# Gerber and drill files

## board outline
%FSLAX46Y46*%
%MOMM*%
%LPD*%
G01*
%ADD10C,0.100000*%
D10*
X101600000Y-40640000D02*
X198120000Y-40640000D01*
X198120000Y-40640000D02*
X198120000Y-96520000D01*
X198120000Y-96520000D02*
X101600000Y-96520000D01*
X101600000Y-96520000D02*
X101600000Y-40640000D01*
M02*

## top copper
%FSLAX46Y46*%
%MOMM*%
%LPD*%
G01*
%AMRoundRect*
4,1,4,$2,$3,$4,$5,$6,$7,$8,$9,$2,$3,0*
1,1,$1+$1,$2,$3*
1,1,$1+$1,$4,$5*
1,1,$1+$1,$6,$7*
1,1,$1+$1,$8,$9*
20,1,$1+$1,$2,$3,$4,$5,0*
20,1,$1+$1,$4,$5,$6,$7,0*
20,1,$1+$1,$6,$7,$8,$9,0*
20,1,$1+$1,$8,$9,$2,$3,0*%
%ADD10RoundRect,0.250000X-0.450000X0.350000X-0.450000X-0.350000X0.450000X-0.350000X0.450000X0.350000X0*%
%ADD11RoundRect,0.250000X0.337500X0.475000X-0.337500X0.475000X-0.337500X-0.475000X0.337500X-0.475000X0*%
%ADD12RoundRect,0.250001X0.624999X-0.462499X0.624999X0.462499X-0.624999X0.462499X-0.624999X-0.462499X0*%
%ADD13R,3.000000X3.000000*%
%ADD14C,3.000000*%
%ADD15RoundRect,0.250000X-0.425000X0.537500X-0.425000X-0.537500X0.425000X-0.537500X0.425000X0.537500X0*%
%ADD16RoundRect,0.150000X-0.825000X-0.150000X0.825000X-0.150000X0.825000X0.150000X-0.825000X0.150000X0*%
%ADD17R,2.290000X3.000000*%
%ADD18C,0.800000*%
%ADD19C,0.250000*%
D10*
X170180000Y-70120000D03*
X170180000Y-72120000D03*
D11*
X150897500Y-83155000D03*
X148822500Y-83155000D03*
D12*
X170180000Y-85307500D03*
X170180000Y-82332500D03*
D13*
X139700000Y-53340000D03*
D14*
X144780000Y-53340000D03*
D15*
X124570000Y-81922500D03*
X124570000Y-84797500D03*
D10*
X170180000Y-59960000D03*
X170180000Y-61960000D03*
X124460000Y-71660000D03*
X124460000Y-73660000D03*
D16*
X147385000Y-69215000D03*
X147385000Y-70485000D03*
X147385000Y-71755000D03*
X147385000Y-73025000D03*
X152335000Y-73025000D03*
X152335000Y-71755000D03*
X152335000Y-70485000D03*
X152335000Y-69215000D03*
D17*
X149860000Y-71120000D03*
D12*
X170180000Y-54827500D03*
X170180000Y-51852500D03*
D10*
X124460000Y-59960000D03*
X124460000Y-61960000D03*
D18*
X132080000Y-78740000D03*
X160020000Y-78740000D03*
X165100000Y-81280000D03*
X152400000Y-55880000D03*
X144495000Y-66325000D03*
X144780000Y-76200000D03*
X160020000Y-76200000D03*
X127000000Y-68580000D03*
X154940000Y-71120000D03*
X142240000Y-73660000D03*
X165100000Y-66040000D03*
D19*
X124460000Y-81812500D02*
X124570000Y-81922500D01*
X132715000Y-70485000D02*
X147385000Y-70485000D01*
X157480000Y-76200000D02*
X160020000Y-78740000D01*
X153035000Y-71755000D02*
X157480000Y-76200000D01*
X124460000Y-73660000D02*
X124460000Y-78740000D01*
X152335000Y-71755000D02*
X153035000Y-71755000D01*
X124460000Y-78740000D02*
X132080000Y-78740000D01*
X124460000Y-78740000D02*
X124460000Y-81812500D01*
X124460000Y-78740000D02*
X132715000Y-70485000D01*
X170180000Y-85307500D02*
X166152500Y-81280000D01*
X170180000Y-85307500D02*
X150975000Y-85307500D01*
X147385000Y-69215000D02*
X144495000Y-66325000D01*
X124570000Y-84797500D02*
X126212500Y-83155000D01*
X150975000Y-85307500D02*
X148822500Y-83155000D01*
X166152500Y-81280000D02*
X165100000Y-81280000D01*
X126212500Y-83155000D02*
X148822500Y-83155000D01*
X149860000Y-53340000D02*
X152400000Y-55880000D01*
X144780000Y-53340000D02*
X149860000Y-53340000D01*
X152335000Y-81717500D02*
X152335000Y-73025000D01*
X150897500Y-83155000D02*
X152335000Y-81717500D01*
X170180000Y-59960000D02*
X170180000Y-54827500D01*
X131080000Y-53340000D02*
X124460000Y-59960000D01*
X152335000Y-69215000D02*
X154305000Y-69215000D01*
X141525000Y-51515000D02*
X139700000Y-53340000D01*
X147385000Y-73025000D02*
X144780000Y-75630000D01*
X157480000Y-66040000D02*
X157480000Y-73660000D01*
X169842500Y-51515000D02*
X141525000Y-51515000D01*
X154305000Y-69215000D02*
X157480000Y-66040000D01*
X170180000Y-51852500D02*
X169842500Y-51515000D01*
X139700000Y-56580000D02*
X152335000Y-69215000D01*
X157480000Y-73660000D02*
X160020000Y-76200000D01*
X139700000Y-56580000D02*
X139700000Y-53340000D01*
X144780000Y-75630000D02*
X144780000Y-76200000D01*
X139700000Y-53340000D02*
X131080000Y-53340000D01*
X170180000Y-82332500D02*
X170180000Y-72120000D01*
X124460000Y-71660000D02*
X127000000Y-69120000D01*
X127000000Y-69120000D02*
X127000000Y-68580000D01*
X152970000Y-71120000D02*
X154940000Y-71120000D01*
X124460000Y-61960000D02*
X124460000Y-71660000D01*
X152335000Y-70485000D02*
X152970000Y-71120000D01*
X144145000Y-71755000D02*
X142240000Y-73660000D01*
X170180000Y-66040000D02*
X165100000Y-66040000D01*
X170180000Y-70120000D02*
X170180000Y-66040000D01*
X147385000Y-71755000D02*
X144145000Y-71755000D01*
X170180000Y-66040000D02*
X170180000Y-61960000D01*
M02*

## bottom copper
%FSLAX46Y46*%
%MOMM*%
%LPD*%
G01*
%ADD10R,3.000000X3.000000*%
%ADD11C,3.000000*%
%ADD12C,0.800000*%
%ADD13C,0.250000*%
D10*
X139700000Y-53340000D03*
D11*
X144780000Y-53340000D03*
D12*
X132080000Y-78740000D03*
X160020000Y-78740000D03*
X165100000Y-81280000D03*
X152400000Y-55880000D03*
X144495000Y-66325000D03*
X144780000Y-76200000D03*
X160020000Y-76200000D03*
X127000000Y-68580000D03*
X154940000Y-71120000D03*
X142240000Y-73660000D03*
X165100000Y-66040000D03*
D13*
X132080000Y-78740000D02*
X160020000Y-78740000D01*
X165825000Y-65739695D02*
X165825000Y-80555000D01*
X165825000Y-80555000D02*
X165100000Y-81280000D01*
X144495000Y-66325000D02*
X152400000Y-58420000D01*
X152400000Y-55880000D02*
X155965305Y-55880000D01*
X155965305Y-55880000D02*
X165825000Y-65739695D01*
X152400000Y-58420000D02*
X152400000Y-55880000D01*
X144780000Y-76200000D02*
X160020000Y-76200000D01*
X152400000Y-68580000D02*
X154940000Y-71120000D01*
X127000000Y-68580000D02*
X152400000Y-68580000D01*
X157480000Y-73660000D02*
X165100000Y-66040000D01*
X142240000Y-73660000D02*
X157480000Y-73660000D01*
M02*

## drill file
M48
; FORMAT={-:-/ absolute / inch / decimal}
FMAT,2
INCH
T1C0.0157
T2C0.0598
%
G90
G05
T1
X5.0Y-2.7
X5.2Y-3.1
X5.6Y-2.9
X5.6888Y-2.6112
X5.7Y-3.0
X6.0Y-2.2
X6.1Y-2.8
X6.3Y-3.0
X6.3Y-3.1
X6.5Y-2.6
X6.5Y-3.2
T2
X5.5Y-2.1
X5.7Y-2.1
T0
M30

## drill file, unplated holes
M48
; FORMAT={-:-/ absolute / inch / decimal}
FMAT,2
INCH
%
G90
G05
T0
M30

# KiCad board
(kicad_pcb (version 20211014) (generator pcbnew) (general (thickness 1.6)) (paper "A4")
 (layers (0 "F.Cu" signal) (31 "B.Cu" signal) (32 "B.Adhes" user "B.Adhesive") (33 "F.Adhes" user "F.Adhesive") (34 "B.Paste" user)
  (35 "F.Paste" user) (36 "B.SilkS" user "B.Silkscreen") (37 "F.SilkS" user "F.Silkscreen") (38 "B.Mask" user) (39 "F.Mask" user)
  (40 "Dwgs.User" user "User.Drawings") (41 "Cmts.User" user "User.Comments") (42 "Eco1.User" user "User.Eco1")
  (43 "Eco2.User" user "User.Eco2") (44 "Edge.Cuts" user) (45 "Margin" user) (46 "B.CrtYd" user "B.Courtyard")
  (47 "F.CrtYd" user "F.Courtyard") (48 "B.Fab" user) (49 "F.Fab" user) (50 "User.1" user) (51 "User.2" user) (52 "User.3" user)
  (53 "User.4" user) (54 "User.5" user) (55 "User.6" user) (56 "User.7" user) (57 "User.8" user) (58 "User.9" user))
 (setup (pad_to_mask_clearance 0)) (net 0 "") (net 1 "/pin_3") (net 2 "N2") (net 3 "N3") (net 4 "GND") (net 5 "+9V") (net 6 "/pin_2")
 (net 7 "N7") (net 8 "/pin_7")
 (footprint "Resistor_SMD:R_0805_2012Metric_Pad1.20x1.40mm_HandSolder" (layer "F.Cu") (at 170.18 71.12 -90)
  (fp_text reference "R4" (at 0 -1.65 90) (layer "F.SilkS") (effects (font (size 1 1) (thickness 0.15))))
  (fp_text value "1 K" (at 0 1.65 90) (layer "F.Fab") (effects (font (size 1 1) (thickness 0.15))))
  (pad "1" smd roundrect (at -1 0 270) (size 1.2 1.4) (layers "F.Cu" "F.Paste" "F.Mask") (roundrect_rratio 0.2083333333) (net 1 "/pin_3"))
  (pad "2" smd roundrect (at 1 0 270) (size 1.2 1.4) (layers "F.Cu" "F.Paste" "F.Mask") (roundrect_rratio 0.2083333333) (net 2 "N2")))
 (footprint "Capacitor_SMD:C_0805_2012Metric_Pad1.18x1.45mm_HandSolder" (layer "F.Cu") (at 149.86 83.155 180)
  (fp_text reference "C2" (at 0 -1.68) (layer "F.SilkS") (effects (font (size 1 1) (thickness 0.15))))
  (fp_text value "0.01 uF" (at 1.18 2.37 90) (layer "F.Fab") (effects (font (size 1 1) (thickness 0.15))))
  (pad "1" smd roundrect (at -1.0375 0 180) (size 1.175 1.45) (layers "F.Cu" "F.Paste" "F.Mask") (roundrect_rratio 0.2127659574)
   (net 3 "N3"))
  (pad "2" smd roundrect (at 1.0375 0 180) (size 1.175 1.45) (layers "F.Cu" "F.Paste" "F.Mask") (roundrect_rratio 0.2127659574)
   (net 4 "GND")))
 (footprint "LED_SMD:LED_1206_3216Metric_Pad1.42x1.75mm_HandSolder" (layer "F.Cu") (at 170.18 83.82 90)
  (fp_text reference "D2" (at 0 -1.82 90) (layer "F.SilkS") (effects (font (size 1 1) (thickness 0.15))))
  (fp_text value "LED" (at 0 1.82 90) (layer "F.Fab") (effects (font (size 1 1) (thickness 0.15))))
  (pad "1" smd roundrect (at -1.4875 0 90) (size 1.425 1.75) (layers "F.Cu" "F.Paste" "F.Mask") (roundrect_rratio 0.1754392982)
   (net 4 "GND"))
  (pad "2" smd roundrect (at 1.4875 0 90) (size 1.425 1.75) (layers "F.Cu" "F.Paste" "F.Mask") (roundrect_rratio 0.1754392982) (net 2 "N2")))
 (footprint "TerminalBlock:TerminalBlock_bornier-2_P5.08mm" (layer "F.Cu") (at 139.7 53.34)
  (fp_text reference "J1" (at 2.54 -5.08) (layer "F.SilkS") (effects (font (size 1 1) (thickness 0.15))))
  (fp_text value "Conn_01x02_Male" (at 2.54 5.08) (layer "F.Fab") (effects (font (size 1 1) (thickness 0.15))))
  (pad "1" thru_hole rect (at 0 0) (size 3 3) (drill 1.52) (layers *.Cu *.Mask) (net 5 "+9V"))
  (pad "2" thru_hole circle (at 5.08 0) (size 3 3) (drill 1.52) (layers *.Cu *.Mask) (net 4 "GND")))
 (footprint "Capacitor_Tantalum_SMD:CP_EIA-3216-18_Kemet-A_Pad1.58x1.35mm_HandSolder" (layer "F.Cu") (at 124.57 83.36 -90)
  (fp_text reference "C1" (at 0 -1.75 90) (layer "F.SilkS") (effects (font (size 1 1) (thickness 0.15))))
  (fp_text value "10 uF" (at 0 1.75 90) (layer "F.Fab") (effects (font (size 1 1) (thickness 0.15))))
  (pad "1" smd roundrect (at -1.4375 0 270) (size 1.575 1.35) (layers "F.Cu" "F.Paste" "F.Mask") (roundrect_rratio 0.1851851852)
   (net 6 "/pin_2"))
  (pad "2" smd roundrect (at 1.4375 0 270) (size 1.575 1.35) (layers "F.Cu" "F.Paste" "F.Mask") (roundrect_rratio 0.1851851852)
   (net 4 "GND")))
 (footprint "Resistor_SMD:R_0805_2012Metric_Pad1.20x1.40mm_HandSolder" (layer "F.Cu") (at 170.18 60.96 -90)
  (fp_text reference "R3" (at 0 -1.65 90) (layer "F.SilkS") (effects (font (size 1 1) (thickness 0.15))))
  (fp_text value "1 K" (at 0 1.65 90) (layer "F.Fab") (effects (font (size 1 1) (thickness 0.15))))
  (pad "1" smd roundrect (at -1 0 270) (size 1.2 1.4) (layers "F.Cu" "F.Paste" "F.Mask") (roundrect_rratio 0.2083333333) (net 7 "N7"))
  (pad "2" smd roundrect (at 1 0 270) (size 1.2 1.4) (layers "F.Cu" "F.Paste" "F.Mask") (roundrect_rratio 0.2083333333) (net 1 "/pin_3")))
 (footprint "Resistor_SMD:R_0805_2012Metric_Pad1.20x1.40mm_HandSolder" (layer "F.Cu") (at 124.46 72.66 -90)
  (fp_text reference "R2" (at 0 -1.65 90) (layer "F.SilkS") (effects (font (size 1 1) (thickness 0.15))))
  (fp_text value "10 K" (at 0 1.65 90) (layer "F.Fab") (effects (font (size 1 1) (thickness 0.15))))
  (pad "1" smd roundrect (at -1 0 270) (size 1.2 1.4) (layers "F.Cu" "F.Paste" "F.Mask") (roundrect_rratio 0.2083333333) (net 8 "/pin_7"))
  (pad "2" smd roundrect (at 1 0 270) (size 1.2 1.4) (layers "F.Cu" "F.Paste" "F.Mask") (roundrect_rratio 0.2083333333) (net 6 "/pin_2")))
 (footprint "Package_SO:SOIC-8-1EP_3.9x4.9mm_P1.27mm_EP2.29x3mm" (layer "F.Cu") (at 149.86 71.12)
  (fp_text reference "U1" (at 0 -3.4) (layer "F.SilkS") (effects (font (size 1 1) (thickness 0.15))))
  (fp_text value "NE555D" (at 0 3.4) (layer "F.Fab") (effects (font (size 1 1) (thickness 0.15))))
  (pad "" smd roundrect (at -0.57 -0.75) (size 0.92 1.21) (layers "F.Paste") (roundrect_rratio 0.25))
  (pad "" smd roundrect (at 0.57 0.75) (size 0.92 1.21) (layers "F.Paste") (roundrect_rratio 0.25))
  (pad "" smd roundrect (at 0.57 -0.75) (size 0.92 1.21) (layers "F.Paste") (roundrect_rratio 0.25))
  (pad "" smd roundrect (at -0.57 0.75) (size 0.92 1.21) (layers "F.Paste") (roundrect_rratio 0.25))
  (pad "1" smd roundrect (at -2.475 -1.905) (size 1.95 0.6) (layers "F.Cu" "F.Paste" "F.Mask") (roundrect_rratio 0.25) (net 4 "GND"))
  (pad "2" smd roundrect (at -2.475 -0.635) (size 1.95 0.6) (layers "F.Cu" "F.Paste" "F.Mask") (roundrect_rratio 0.25) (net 6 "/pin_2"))
  (pad "3" smd roundrect (at -2.475 0.635) (size 1.95 0.6) (layers "F.Cu" "F.Paste" "F.Mask") (roundrect_rratio 0.25) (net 1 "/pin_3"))
  (pad "4" smd roundrect (at -2.475 1.905) (size 1.95 0.6) (layers "F.Cu" "F.Paste" "F.Mask") (roundrect_rratio 0.25) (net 5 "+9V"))
  (pad "5" smd roundrect (at 2.475 1.905) (size 1.95 0.6) (layers "F.Cu" "F.Paste" "F.Mask") (roundrect_rratio 0.25) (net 3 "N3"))
  (pad "6" smd roundrect (at 2.475 0.635) (size 1.95 0.6) (layers "F.Cu" "F.Paste" "F.Mask") (roundrect_rratio 0.25) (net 6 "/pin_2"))
  (pad "7" smd roundrect (at 2.475 -0.635) (size 1.95 0.6) (layers "F.Cu" "F.Paste" "F.Mask") (roundrect_rratio 0.25) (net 8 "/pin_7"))
  (pad "8" smd roundrect (at 2.475 -1.905) (size 1.95 0.6) (layers "F.Cu" "F.Paste" "F.Mask") (roundrect_rratio 0.25) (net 5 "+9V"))
  (pad "9" smd rect (at 0 0) (size 2.29 3) (layers "F.Cu" "F.Mask")))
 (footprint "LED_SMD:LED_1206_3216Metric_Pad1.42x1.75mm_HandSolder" (layer "F.Cu") (at 170.18 53.34 90)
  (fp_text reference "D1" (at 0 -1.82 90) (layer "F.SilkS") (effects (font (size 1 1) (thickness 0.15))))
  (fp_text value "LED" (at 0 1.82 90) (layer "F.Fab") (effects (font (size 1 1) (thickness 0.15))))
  (pad "1" smd roundrect (at -1.4875 0 90) (size 1.425 1.75) (layers "F.Cu" "F.Paste" "F.Mask") (roundrect_rratio 0.1754392982) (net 7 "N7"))
  (pad "2" smd roundrect (at 1.4875 0 90) (size 1.425 1.75) (layers "F.Cu" "F.Paste" "F.Mask") (roundrect_rratio 0.1754392982) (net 5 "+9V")))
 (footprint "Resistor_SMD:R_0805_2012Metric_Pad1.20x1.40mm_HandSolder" (layer "F.Cu") (at 124.46 60.96 -90)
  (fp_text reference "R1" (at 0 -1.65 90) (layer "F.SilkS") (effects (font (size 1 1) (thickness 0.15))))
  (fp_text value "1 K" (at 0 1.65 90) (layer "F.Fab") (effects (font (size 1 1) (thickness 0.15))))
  (pad "1" smd roundrect (at -1 0 270) (size 1.2 1.4) (layers "F.Cu" "F.Paste" "F.Mask") (roundrect_rratio 0.2083333333) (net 5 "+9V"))
  (pad "2" smd roundrect (at 1 0 270) (size 1.2 1.4) (layers "F.Cu" "F.Paste" "F.Mask") (roundrect_rratio 0.2083333333) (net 8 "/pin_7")))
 (gr_rect (start 101.6 40.64) (end 198.12 96.52) (layer "Edge.Cuts") (width 0.1) (fill none))
 (segment (start 124.46 81.8125) (end 124.57 81.9225) (width 0.25) (layer "F.Cu") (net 6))
 (segment (start 132.715 70.485) (end 147.385 70.485) (width 0.25) (layer "F.Cu") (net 6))
 (segment (start 157.48 76.2) (end 160.02 78.74) (width 0.25) (layer "F.Cu") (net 6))
 (segment (start 153.035 71.755) (end 157.48 76.2) (width 0.25) (layer "F.Cu") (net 6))
 (segment (start 124.46 73.66) (end 124.46 78.74) (width 0.25) (layer "F.Cu") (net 6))
 (segment (start 152.335 71.755) (end 153.035 71.755) (width 0.25) (layer "F.Cu") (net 6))
 (segment (start 124.46 78.74) (end 132.08 78.74) (width 0.25) (layer "F.Cu") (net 6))
 (segment (start 124.46 78.74) (end 124.46 81.8125) (width 0.25) (layer "F.Cu") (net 6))
 (segment (start 124.46 78.74) (end 132.715 70.485) (width 0.25) (layer "F.Cu") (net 6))
 (via (at 132.08 78.74) (size 0.8) (drill 0.4) (layers "F.Cu" "B.Cu") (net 6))
 (via (at 160.02 78.74) (size 0.8) (drill 0.4) (layers "F.Cu" "B.Cu") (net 6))
 (segment (start 132.08 78.74) (end 160.02 78.74) (width 0.25) (layer "B.Cu") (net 6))
 (segment (start 170.18 85.3075) (end 166.1525 81.28) (width 0.25) (layer "F.Cu") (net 4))
 (segment (start 170.18 85.3075) (end 150.975 85.3075) (width 0.25) (layer "F.Cu") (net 4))
 (segment (start 147.385 69.215) (end 144.495 66.325) (width 0.25) (layer "F.Cu") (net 4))
 (segment (start 124.57 84.7975) (end 126.2125 83.155) (width 0.25) (layer "F.Cu") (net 4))
 (segment (start 150.975 85.3075) (end 148.8225 83.155) (width 0.25) (layer "F.Cu") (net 4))
 (segment (start 166.1525 81.28) (end 165.1 81.28) (width 0.25) (layer "F.Cu") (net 4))
 (segment (start 126.2125 83.155) (end 148.8225 83.155) (width 0.25) (layer "F.Cu") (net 4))
 (segment (start 149.86 53.34) (end 152.4 55.88) (width 0.25) (layer "F.Cu") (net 4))
 (segment (start 144.78 53.34) (end 149.86 53.34) (width 0.25) (layer "F.Cu") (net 4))
 (via (at 165.1 81.28) (size 0.8) (drill 0.4) (layers "F.Cu" "B.Cu") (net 4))
 (via (at 152.4 55.88) (size 0.8) (drill 0.4) (layers "F.Cu" "B.Cu") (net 4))
 (via (at 144.495 66.325) (size 0.8) (drill 0.4) (layers "F.Cu" "B.Cu") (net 4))
 (segment (start 165.825 65.739695) (end 165.825 80.555) (width 0.25) (layer "B.Cu") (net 4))
 (segment (start 165.825 80.555) (end 165.1 81.28) (width 0.25) (layer "B.Cu") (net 4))
 (segment (start 144.495 66.325) (end 152.4 58.42) (width 0.25) (layer "B.Cu") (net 4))
 (segment (start 152.4 55.88) (end 155.965305 55.88) (width 0.25) (layer "B.Cu") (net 4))
 (segment (start 155.965305 55.88) (end 165.825 65.739695) (width 0.25) (layer "B.Cu") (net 4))
 (segment (start 152.4 58.42) (end 152.4 55.88) (width 0.25) (layer "B.Cu") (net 4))
 (segment (start 152.335 81.7175) (end 152.335 73.025) (width 0.25) (layer "F.Cu") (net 3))
 (segment (start 150.8975 83.155) (end 152.335 81.7175) (width 0.25) (layer "F.Cu") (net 3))
 (segment (start 170.18 59.96) (end 170.18 54.8275) (width 0.25) (layer "F.Cu") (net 7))
 (segment (start 131.08 53.34) (end 124.46 59.96) (width 0.25) (layer "F.Cu") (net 5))
 (segment (start 152.335 69.215) (end 154.305 69.215) (width 0.25) (layer "F.Cu") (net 5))
 (segment (start 141.525 51.515) (end 139.7 53.34) (width 0.25) (layer "F.Cu") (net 5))
 (segment (start 147.385 73.025) (end 144.78 75.63) (width 0.25) (layer "F.Cu") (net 5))
 (segment (start 157.48 66.04) (end 157.48 73.66) (width 0.25) (layer "F.Cu") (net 5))
 (segment (start 169.8425 51.515) (end 141.525 51.515) (width 0.25) (layer "F.Cu") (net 5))
 (segment (start 154.305 69.215) (end 157.48 66.04) (width 0.25) (layer "F.Cu") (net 5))
 (segment (start 170.18 51.8525) (end 169.8425 51.515) (width 0.25) (layer "F.Cu") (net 5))
 (segment (start 139.7 56.58) (end 152.335 69.215) (width 0.25) (layer "F.Cu") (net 5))
 (segment (start 157.48 73.66) (end 160.02 76.2) (width 0.25) (layer "F.Cu") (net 5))
 (segment (start 139.7 56.58) (end 139.7 53.34) (width 0.25) (layer "F.Cu") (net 5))
 (segment (start 144.78 75.63) (end 144.78 76.2) (width 0.25) (layer "F.Cu") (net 5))
 (segment (start 139.7 53.34) (end 131.08 53.34) (width 0.25) (layer "F.Cu") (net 5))
 (via (at 144.78 76.2) (size 0.8) (drill 0.4) (layers "F.Cu" "B.Cu") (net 5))
 (via (at 160.02 76.2) (size 0.8) (drill 0.4) (layers "F.Cu" "B.Cu") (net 5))
 (segment (start 144.78 76.2) (end 160.02 76.2) (width 0.25) (layer "B.Cu") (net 5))
 (segment (start 170.18 82.3325) (end 170.18 72.12) (width 0.25) (layer "F.Cu") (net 2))
 (segment (start 124.46 71.66) (end 127 69.12) (width 0.25) (layer "F.Cu") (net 8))
 (segment (start 127 69.12) (end 127 68.58) (width 0.25) (layer "F.Cu") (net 8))
 (segment (start 152.97 71.12) (end 154.94 71.12) (width 0.25) (layer "F.Cu") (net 8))
 (segment (start 124.46 61.96) (end 124.46 71.66) (width 0.25) (layer "F.Cu") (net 8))
 (segment (start 152.335 70.485) (end 152.97 71.12) (width 0.25) (layer "F.Cu") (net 8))
 (via (at 127 68.58) (size 0.8) (drill 0.4) (layers "F.Cu" "B.Cu") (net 8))
 (via (at 154.94 71.12) (size 0.8) (drill 0.4) (layers "F.Cu" "B.Cu") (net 8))
 (segment (start 152.4 68.58) (end 154.94 71.12) (width 0.25) (layer "B.Cu") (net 8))
 (segment (start 127 68.58) (end 152.4 68.58) (width 0.25) (layer "B.Cu") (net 8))
 (segment (start 144.145 71.755) (end 142.24 73.66) (width 0.25) (layer "F.Cu") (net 1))
 (segment (start 170.18 66.04) (end 165.1 66.04) (width 0.25) (layer "F.Cu") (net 1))
 (segment (start 170.18 70.12) (end 170.18 66.04) (width 0.25) (layer "F.Cu") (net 1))
 (segment (start 147.385 71.755) (end 144.145 71.755) (width 0.25) (layer "F.Cu") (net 1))
 (segment (start 170.18 66.04) (end 170.18 61.96) (width 0.25) (layer "F.Cu") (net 1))
 (via (at 142.24 73.66) (size 0.8) (drill 0.4) (layers "F.Cu" "B.Cu") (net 1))
 (via (at 165.1 66.04) (size 0.8) (drill 0.4) (layers "F.Cu" "B.Cu") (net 1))
 (segment (start 157.48 73.66) (end 165.1 66.04) (width 0.25) (layer "B.Cu") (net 1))
 (segment (start 142.24 73.66) (end 157.48 73.66) (width 0.25) (layer "B.Cu") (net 1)))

